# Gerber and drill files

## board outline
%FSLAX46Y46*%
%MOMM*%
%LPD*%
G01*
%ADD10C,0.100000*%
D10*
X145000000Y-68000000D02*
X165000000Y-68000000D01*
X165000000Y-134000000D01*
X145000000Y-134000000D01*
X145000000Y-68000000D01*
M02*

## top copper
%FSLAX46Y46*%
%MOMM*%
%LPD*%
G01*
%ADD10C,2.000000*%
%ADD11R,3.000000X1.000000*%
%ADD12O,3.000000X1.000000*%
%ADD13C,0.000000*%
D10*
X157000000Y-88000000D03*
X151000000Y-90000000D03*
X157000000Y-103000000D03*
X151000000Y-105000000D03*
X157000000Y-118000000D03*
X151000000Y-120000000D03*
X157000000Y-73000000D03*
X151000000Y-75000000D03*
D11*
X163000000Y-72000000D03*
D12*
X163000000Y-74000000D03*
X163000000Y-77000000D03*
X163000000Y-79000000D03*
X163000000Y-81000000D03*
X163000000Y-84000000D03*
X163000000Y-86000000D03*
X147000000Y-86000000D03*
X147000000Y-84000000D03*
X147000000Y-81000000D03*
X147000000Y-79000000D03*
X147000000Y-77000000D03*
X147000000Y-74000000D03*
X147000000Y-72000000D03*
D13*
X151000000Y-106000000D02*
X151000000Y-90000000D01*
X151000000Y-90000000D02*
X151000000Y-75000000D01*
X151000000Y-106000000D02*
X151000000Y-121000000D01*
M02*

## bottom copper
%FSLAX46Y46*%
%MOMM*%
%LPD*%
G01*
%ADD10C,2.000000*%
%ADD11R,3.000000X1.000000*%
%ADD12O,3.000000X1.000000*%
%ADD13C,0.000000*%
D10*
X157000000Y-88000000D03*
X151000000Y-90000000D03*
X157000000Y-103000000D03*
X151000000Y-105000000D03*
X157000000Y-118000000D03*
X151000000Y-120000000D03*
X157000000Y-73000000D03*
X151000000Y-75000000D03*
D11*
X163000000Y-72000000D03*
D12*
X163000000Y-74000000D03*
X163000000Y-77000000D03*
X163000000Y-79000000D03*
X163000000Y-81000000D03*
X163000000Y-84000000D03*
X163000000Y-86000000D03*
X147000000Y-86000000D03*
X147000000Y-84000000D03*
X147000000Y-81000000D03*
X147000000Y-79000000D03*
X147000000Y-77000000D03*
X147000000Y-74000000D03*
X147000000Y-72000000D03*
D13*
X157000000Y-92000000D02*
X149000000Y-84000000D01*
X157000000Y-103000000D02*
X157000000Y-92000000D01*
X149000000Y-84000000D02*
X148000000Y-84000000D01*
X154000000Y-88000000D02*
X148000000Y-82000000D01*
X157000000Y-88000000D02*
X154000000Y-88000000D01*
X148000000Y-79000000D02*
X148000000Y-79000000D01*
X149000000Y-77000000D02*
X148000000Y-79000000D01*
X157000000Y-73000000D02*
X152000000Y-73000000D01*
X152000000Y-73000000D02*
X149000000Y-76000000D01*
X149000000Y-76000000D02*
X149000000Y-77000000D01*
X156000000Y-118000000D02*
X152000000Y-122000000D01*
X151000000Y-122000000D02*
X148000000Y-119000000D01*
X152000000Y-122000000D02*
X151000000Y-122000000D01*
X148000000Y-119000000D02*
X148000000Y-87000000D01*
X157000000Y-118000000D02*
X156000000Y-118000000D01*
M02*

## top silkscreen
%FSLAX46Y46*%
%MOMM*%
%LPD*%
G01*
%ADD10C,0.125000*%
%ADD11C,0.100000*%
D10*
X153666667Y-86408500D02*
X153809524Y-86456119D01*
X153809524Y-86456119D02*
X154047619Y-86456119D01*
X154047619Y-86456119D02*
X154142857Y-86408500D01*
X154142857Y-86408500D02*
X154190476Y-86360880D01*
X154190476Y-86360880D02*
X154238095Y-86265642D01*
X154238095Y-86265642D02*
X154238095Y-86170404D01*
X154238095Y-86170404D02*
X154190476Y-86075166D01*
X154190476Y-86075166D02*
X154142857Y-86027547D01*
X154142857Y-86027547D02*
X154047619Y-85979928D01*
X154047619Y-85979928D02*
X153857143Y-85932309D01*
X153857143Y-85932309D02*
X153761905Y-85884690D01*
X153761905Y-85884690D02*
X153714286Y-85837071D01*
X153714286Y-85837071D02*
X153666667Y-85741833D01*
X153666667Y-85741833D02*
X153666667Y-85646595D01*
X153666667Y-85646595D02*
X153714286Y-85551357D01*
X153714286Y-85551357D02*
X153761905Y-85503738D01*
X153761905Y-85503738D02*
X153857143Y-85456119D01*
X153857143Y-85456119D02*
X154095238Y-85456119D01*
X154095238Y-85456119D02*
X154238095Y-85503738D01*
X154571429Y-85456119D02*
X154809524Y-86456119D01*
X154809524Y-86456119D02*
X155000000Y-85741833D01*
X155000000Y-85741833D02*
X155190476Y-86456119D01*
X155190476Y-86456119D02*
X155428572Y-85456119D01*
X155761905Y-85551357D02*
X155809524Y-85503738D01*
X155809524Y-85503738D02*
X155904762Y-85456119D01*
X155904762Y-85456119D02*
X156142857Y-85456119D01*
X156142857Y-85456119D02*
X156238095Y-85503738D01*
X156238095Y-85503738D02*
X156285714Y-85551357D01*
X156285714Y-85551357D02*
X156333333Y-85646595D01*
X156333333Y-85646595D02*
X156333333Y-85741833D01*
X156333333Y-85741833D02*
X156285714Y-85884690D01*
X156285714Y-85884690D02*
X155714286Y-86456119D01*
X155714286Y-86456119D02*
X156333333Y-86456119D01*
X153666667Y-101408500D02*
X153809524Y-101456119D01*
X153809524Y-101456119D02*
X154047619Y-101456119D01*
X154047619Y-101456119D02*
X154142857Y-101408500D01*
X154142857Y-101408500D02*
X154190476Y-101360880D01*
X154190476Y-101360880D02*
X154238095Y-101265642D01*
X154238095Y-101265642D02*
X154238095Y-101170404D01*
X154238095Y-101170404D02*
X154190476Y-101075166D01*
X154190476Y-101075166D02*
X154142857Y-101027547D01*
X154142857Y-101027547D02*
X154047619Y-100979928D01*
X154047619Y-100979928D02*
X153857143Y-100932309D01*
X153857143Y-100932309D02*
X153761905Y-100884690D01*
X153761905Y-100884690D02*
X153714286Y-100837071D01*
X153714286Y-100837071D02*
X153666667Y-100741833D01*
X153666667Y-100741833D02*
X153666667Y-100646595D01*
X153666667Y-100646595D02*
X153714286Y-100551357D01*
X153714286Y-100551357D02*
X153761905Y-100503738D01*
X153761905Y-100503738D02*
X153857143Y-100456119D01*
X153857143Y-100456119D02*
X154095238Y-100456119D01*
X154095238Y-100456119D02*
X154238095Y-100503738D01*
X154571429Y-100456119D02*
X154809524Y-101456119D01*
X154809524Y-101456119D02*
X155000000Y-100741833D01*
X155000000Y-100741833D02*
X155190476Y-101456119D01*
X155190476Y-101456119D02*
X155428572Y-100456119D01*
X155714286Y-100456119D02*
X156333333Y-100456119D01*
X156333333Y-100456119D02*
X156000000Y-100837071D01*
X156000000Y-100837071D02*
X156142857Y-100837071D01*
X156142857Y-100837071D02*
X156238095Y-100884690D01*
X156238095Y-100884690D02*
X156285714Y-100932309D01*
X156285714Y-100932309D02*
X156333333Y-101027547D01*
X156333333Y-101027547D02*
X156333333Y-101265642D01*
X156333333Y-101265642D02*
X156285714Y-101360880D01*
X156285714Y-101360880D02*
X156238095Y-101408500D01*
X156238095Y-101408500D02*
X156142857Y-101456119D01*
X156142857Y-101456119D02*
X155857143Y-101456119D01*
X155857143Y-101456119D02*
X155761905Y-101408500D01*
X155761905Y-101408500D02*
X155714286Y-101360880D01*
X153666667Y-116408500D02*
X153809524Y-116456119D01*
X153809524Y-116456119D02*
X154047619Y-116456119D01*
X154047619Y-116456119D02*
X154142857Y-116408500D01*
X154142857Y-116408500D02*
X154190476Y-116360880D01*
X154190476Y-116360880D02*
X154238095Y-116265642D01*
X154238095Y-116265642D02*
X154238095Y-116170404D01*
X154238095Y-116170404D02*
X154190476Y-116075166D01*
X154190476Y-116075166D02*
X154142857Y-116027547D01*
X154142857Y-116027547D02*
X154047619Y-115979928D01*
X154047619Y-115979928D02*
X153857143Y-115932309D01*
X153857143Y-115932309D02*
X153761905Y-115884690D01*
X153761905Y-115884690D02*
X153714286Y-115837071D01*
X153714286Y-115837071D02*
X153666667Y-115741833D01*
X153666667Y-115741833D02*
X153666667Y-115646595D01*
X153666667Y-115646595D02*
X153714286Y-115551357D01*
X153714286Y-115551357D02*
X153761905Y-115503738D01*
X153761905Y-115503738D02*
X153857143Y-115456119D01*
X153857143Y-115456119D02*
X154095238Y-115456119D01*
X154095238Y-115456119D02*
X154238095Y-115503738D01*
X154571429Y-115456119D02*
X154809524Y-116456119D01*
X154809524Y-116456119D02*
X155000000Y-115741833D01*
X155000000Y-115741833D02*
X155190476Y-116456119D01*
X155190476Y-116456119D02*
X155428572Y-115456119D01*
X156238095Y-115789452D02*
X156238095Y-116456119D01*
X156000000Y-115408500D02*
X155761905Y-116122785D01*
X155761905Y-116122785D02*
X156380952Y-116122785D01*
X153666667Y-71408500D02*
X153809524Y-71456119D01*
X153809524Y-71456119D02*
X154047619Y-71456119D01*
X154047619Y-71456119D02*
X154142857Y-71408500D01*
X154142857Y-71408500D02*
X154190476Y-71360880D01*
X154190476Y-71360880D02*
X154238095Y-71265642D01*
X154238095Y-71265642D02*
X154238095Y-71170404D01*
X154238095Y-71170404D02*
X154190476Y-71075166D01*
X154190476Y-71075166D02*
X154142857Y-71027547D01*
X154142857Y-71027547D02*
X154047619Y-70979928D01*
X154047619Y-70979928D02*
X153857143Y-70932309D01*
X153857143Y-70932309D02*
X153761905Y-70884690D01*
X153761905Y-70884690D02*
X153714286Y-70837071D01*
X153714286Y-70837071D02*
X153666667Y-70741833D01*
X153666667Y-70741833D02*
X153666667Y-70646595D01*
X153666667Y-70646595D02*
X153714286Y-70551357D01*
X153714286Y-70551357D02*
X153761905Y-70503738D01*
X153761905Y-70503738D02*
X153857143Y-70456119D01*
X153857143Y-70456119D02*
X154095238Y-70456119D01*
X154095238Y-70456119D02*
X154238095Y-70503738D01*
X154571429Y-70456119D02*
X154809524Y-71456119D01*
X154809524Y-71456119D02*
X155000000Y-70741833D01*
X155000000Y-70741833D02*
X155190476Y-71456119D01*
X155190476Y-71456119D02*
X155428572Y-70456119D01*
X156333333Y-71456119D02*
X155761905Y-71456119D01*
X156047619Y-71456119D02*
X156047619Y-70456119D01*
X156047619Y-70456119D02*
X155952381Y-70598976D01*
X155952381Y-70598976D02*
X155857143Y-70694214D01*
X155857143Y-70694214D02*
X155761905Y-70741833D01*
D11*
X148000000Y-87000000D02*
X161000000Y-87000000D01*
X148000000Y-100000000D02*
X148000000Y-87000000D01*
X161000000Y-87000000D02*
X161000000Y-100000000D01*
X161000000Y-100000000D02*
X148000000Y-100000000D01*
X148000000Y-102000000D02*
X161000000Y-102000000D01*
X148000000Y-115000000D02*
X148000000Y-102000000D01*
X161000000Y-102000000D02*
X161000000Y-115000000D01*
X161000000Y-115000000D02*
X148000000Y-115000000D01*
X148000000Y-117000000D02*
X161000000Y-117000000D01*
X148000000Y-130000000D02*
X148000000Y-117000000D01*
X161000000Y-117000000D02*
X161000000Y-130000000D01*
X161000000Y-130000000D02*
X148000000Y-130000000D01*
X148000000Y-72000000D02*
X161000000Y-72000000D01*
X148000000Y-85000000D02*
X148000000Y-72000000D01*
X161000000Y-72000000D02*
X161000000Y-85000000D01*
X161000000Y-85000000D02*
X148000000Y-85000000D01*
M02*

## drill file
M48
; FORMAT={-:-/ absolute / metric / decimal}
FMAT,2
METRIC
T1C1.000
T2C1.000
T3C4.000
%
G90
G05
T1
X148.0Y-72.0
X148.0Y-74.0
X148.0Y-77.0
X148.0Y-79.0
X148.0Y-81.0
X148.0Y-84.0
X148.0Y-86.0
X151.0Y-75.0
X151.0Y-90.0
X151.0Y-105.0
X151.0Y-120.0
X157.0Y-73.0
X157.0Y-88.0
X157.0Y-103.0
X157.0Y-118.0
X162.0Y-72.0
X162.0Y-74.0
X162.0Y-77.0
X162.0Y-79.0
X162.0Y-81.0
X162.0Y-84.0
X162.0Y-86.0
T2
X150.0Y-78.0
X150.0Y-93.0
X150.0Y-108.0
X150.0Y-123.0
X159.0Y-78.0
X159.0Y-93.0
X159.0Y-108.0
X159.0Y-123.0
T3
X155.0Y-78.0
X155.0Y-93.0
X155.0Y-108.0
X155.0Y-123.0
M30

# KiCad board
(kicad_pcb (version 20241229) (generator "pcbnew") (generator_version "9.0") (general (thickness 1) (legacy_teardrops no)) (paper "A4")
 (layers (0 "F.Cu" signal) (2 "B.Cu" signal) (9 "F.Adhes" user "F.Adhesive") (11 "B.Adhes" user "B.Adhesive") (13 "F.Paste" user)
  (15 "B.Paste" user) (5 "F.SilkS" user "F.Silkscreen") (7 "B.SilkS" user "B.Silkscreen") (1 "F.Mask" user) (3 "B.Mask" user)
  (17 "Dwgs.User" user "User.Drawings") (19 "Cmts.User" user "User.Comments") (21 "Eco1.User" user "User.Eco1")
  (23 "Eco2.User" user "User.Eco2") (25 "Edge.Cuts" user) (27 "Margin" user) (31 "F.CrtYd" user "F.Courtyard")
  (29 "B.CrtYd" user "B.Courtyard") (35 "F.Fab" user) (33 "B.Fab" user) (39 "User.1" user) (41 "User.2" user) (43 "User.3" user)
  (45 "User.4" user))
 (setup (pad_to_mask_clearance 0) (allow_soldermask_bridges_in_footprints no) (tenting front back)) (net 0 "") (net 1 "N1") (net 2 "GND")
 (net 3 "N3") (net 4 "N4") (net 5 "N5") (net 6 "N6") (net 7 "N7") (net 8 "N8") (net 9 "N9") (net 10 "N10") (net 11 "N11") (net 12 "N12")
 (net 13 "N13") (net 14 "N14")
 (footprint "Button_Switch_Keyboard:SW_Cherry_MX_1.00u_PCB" (layer "F.Cu") (at 157 88)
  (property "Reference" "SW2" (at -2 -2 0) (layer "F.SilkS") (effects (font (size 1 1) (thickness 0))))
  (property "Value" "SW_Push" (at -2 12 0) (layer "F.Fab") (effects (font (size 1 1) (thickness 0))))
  (fp_line (start -9 -1) (end 4 -1) (stroke (width 0) (type solid)) (layer "F.SilkS"))
  (fp_line (start -9 12) (end -9 -1) (stroke (width 0) (type solid)) (layer "F.SilkS"))
  (fp_line (start 4 -1) (end 4 12) (stroke (width 0) (type solid)) (layer "F.SilkS"))
  (fp_line (start 4 12) (end -9 12) (stroke (width 0) (type solid)) (layer "F.SilkS"))
  (pad "" np_thru_hole circle (at -7 5) (size 1 1) (drill 1) (layers "*.Cu" "*.Mask"))
  (pad "" np_thru_hole circle (at -2 5) (size 4 4) (drill 4) (layers "*.Cu" "*.Mask"))
  (pad "" np_thru_hole circle (at 2 5) (size 1 1) (drill 1) (layers "*.Cu" "*.Mask"))
  (pad "1" thru_hole circle (at 0 0) (size 2 2) (drill 1) (layers "*.Cu" "*.Mask") (remove_unused_layers no) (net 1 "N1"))
  (pad "2" thru_hole circle (at -6 2) (size 2 2) (drill 1) (layers "*.Cu" "*.Mask") (remove_unused_layers no) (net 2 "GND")))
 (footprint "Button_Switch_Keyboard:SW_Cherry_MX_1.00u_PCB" (layer "F.Cu") (at 157 103)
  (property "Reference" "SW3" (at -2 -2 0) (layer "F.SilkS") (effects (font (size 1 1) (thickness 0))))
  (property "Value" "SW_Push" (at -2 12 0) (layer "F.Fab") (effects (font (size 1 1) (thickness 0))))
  (fp_line (start -9 -1) (end 4 -1) (stroke (width 0) (type solid)) (layer "F.SilkS"))
  (fp_line (start -9 12) (end -9 -1) (stroke (width 0) (type solid)) (layer "F.SilkS"))
  (fp_line (start 4 -1) (end 4 12) (stroke (width 0) (type solid)) (layer "F.SilkS"))
  (fp_line (start 4 12) (end -9 12) (stroke (width 0) (type solid)) (layer "F.SilkS"))
  (pad "" np_thru_hole circle (at -7 5) (size 1 1) (drill 1) (layers "*.Cu" "*.Mask"))
  (pad "" np_thru_hole circle (at -2 5) (size 4 4) (drill 4) (layers "*.Cu" "*.Mask"))
  (pad "" np_thru_hole circle (at 2 5) (size 1 1) (drill 1) (layers "*.Cu" "*.Mask"))
  (pad "1" thru_hole circle (at 0 0) (size 2 2) (drill 1) (layers "*.Cu" "*.Mask") (remove_unused_layers no) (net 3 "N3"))
  (pad "2" thru_hole circle (at -6 2) (size 2 2) (drill 1) (layers "*.Cu" "*.Mask") (remove_unused_layers no) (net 2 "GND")))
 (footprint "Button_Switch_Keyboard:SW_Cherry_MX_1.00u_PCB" (layer "F.Cu") (at 157 118)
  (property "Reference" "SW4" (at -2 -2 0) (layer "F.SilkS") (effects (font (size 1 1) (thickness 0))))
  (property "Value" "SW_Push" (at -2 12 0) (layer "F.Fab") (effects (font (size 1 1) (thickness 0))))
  (fp_line (start -9 -1) (end 4 -1) (stroke (width 0) (type solid)) (layer "F.SilkS"))
  (fp_line (start -9 12) (end -9 -1) (stroke (width 0) (type solid)) (layer "F.SilkS"))
  (fp_line (start 4 -1) (end 4 12) (stroke (width 0) (type solid)) (layer "F.SilkS"))
  (fp_line (start 4 12) (end -9 12) (stroke (width 0) (type solid)) (layer "F.SilkS"))
  (pad "" np_thru_hole circle (at -7 5) (size 1 1) (drill 1) (layers "*.Cu" "*.Mask"))
  (pad "" np_thru_hole circle (at -2 5) (size 4 4) (drill 4) (layers "*.Cu" "*.Mask"))
  (pad "" np_thru_hole circle (at 2 5) (size 1 1) (drill 1) (layers "*.Cu" "*.Mask"))
  (pad "1" thru_hole circle (at 0 0) (size 2 2) (drill 1) (layers "*.Cu" "*.Mask") (remove_unused_layers no) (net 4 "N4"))
  (pad "2" thru_hole circle (at -6 2) (size 2 2) (drill 1) (layers "*.Cu" "*.Mask") (remove_unused_layers no) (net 2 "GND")))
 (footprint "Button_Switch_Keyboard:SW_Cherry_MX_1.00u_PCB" (layer "F.Cu") (at 157 73)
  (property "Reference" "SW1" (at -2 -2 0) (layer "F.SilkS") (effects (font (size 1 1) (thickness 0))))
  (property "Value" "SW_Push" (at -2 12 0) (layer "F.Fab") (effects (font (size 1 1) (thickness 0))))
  (fp_line (start -9 -1) (end 4 -1) (stroke (width 0) (type solid)) (layer "F.SilkS"))
  (fp_line (start -9 12) (end -9 -1) (stroke (width 0) (type solid)) (layer "F.SilkS"))
  (fp_line (start 4 -1) (end 4 12) (stroke (width 0) (type solid)) (layer "F.SilkS"))
  (fp_line (start 4 12) (end -9 12) (stroke (width 0) (type solid)) (layer "F.SilkS"))
  (pad "" np_thru_hole circle (at -7 5) (size 1 1) (drill 1) (layers "*.Cu" "*.Mask"))
  (pad "" np_thru_hole circle (at -2 5) (size 4 4) (drill 4) (layers "*.Cu" "*.Mask"))
  (pad "" np_thru_hole circle (at 2 5) (size 1 1) (drill 1) (layers "*.Cu" "*.Mask"))
  (pad "1" thru_hole circle (at 0 0) (size 2 2) (drill 1) (layers "*.Cu" "*.Mask") (remove_unused_layers no) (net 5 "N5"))
  (pad "2" thru_hole circle (at -6 2) (size 2 2) (drill 1) (layers "*.Cu" "*.Mask") (remove_unused_layers no) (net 2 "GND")))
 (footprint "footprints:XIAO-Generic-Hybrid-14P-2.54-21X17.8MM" (layer "B.Cu") (at 155 79 180)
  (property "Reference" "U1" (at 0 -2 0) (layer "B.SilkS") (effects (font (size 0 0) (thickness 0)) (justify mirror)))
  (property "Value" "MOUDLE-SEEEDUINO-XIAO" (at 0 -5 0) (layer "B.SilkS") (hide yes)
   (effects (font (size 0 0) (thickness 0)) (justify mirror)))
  (pad "1" thru_hole rect (at -7 7 180) (size 3 1) (drill 1 (offset -1 0)) (layers "*.Cu" "*.Mask") (remove_unused_layers no) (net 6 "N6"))
  (pad "2" thru_hole oval (at -7 5 180) (size 3 1) (drill 1 (offset -1 0)) (layers "*.Cu" "*.Mask") (remove_unused_layers no) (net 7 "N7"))
  (pad "3" thru_hole oval (at -7 2 180) (size 3 1) (drill 1 (offset -1 0)) (layers "*.Cu" "*.Mask") (remove_unused_layers no) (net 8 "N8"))
  (pad "4" thru_hole oval (at -7 0 180) (size 3 1) (drill 1 (offset -1 0)) (layers "*.Cu" "*.Mask") (remove_unused_layers no) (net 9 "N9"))
  (pad "5" thru_hole oval (at -7 -2 180) (size 3 1) (drill 1 (offset -1 0)) (layers "*.Cu" "*.Mask") (remove_unused_layers no)
   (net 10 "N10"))
  (pad "6" thru_hole oval (at -7 -5) (size 3 1) (drill 1 (offset 1 0)) (layers "*.Cu" "*.Mask") (remove_unused_layers no) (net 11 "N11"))
  (pad "7" thru_hole oval (at -7 -7 180) (size 3 1) (drill 1 (offset -1 0)) (layers "*.Cu" "*.Mask") (remove_unused_layers no)
   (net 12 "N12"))
  (pad "8" thru_hole oval (at 7 -7 180) (size 3 1) (drill 1 (offset 1 0)) (layers "*.Cu" "*.Mask") (remove_unused_layers no) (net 4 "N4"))
  (pad "9" thru_hole oval (at 7 -5 180) (size 3 1) (drill 1 (offset 1 0)) (layers "*.Cu" "*.Mask") (remove_unused_layers no) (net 3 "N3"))
  (pad "10" thru_hole oval (at 7 -2 180) (size 3 1) (drill 1 (offset 1 0)) (layers "*.Cu" "*.Mask") (remove_unused_layers no) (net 1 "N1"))
  (pad "11" thru_hole oval (at 7 0 180) (size 3 1) (drill 1 (offset 1 0)) (layers "*.Cu" "*.Mask") (remove_unused_layers no) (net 5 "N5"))
  (pad "12" thru_hole oval (at 7 2 180) (size 3 1) (drill 1 (offset 1 0)) (layers "*.Cu" "*.Mask") (remove_unused_layers no) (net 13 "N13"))
  (pad "13" thru_hole oval (at 7 5 180) (size 3 1) (drill 1 (offset 1 0)) (layers "*.Cu" "*.Mask") (remove_unused_layers no) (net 2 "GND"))
  (pad "14" thru_hole oval (at 7 7 180) (size 3 1) (drill 1 (offset 1 0)) (layers "*.Cu" "*.Mask") (remove_unused_layers no) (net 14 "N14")))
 (gr_rect (start 145 68) (end 165 134) (stroke (width 0) (type default)) (fill no) (layer "Edge.Cuts"))
 (segment (start 157 92) (end 149 84) (width 0) (layer "B.Cu") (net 3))
 (segment (start 157 103) (end 157 92) (width 0) (layer "B.Cu") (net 3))
 (segment (start 149 84) (end 148 84) (width 0) (layer "B.Cu") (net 3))
 (segment (start 151 106) (end 151 90) (width 0) (layer "F.Cu") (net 2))
 (segment (start 151 90) (end 151 75) (width 0) (layer "F.Cu") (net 2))
 (segment (start 151 106) (end 151 121) (width 0) (layer "F.Cu") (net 2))
 (segment (start 154 88) (end 148 82) (width 0) (layer "B.Cu") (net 1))
 (segment (start 157 88) (end 154 88) (width 0) (layer "B.Cu") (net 1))
 (segment (start 148 79) (end 148 79) (width 0) (layer "B.Cu") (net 5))
 (segment (start 149 77) (end 148 79) (width 0) (layer "B.Cu") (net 5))
 (segment (start 157 73) (end 152 73) (width 0) (layer "B.Cu") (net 5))
 (segment (start 152 73) (end 149 76) (width 0) (layer "B.Cu") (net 5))
 (segment (start 149 76) (end 149 77) (width 0) (layer "B.Cu") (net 5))
 (segment (start 156 118) (end 152 122) (width 0) (layer "B.Cu") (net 4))
 (segment (start 151 122) (end 148 119) (width 0) (layer "B.Cu") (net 4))
 (segment (start 152 122) (end 151 122) (width 0) (layer "B.Cu") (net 4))
 (segment (start 148 119) (end 148 87) (width 0) (layer "B.Cu") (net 4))
 (segment (start 157 118) (end 156 118) (width 0) (layer "B.Cu") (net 4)))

